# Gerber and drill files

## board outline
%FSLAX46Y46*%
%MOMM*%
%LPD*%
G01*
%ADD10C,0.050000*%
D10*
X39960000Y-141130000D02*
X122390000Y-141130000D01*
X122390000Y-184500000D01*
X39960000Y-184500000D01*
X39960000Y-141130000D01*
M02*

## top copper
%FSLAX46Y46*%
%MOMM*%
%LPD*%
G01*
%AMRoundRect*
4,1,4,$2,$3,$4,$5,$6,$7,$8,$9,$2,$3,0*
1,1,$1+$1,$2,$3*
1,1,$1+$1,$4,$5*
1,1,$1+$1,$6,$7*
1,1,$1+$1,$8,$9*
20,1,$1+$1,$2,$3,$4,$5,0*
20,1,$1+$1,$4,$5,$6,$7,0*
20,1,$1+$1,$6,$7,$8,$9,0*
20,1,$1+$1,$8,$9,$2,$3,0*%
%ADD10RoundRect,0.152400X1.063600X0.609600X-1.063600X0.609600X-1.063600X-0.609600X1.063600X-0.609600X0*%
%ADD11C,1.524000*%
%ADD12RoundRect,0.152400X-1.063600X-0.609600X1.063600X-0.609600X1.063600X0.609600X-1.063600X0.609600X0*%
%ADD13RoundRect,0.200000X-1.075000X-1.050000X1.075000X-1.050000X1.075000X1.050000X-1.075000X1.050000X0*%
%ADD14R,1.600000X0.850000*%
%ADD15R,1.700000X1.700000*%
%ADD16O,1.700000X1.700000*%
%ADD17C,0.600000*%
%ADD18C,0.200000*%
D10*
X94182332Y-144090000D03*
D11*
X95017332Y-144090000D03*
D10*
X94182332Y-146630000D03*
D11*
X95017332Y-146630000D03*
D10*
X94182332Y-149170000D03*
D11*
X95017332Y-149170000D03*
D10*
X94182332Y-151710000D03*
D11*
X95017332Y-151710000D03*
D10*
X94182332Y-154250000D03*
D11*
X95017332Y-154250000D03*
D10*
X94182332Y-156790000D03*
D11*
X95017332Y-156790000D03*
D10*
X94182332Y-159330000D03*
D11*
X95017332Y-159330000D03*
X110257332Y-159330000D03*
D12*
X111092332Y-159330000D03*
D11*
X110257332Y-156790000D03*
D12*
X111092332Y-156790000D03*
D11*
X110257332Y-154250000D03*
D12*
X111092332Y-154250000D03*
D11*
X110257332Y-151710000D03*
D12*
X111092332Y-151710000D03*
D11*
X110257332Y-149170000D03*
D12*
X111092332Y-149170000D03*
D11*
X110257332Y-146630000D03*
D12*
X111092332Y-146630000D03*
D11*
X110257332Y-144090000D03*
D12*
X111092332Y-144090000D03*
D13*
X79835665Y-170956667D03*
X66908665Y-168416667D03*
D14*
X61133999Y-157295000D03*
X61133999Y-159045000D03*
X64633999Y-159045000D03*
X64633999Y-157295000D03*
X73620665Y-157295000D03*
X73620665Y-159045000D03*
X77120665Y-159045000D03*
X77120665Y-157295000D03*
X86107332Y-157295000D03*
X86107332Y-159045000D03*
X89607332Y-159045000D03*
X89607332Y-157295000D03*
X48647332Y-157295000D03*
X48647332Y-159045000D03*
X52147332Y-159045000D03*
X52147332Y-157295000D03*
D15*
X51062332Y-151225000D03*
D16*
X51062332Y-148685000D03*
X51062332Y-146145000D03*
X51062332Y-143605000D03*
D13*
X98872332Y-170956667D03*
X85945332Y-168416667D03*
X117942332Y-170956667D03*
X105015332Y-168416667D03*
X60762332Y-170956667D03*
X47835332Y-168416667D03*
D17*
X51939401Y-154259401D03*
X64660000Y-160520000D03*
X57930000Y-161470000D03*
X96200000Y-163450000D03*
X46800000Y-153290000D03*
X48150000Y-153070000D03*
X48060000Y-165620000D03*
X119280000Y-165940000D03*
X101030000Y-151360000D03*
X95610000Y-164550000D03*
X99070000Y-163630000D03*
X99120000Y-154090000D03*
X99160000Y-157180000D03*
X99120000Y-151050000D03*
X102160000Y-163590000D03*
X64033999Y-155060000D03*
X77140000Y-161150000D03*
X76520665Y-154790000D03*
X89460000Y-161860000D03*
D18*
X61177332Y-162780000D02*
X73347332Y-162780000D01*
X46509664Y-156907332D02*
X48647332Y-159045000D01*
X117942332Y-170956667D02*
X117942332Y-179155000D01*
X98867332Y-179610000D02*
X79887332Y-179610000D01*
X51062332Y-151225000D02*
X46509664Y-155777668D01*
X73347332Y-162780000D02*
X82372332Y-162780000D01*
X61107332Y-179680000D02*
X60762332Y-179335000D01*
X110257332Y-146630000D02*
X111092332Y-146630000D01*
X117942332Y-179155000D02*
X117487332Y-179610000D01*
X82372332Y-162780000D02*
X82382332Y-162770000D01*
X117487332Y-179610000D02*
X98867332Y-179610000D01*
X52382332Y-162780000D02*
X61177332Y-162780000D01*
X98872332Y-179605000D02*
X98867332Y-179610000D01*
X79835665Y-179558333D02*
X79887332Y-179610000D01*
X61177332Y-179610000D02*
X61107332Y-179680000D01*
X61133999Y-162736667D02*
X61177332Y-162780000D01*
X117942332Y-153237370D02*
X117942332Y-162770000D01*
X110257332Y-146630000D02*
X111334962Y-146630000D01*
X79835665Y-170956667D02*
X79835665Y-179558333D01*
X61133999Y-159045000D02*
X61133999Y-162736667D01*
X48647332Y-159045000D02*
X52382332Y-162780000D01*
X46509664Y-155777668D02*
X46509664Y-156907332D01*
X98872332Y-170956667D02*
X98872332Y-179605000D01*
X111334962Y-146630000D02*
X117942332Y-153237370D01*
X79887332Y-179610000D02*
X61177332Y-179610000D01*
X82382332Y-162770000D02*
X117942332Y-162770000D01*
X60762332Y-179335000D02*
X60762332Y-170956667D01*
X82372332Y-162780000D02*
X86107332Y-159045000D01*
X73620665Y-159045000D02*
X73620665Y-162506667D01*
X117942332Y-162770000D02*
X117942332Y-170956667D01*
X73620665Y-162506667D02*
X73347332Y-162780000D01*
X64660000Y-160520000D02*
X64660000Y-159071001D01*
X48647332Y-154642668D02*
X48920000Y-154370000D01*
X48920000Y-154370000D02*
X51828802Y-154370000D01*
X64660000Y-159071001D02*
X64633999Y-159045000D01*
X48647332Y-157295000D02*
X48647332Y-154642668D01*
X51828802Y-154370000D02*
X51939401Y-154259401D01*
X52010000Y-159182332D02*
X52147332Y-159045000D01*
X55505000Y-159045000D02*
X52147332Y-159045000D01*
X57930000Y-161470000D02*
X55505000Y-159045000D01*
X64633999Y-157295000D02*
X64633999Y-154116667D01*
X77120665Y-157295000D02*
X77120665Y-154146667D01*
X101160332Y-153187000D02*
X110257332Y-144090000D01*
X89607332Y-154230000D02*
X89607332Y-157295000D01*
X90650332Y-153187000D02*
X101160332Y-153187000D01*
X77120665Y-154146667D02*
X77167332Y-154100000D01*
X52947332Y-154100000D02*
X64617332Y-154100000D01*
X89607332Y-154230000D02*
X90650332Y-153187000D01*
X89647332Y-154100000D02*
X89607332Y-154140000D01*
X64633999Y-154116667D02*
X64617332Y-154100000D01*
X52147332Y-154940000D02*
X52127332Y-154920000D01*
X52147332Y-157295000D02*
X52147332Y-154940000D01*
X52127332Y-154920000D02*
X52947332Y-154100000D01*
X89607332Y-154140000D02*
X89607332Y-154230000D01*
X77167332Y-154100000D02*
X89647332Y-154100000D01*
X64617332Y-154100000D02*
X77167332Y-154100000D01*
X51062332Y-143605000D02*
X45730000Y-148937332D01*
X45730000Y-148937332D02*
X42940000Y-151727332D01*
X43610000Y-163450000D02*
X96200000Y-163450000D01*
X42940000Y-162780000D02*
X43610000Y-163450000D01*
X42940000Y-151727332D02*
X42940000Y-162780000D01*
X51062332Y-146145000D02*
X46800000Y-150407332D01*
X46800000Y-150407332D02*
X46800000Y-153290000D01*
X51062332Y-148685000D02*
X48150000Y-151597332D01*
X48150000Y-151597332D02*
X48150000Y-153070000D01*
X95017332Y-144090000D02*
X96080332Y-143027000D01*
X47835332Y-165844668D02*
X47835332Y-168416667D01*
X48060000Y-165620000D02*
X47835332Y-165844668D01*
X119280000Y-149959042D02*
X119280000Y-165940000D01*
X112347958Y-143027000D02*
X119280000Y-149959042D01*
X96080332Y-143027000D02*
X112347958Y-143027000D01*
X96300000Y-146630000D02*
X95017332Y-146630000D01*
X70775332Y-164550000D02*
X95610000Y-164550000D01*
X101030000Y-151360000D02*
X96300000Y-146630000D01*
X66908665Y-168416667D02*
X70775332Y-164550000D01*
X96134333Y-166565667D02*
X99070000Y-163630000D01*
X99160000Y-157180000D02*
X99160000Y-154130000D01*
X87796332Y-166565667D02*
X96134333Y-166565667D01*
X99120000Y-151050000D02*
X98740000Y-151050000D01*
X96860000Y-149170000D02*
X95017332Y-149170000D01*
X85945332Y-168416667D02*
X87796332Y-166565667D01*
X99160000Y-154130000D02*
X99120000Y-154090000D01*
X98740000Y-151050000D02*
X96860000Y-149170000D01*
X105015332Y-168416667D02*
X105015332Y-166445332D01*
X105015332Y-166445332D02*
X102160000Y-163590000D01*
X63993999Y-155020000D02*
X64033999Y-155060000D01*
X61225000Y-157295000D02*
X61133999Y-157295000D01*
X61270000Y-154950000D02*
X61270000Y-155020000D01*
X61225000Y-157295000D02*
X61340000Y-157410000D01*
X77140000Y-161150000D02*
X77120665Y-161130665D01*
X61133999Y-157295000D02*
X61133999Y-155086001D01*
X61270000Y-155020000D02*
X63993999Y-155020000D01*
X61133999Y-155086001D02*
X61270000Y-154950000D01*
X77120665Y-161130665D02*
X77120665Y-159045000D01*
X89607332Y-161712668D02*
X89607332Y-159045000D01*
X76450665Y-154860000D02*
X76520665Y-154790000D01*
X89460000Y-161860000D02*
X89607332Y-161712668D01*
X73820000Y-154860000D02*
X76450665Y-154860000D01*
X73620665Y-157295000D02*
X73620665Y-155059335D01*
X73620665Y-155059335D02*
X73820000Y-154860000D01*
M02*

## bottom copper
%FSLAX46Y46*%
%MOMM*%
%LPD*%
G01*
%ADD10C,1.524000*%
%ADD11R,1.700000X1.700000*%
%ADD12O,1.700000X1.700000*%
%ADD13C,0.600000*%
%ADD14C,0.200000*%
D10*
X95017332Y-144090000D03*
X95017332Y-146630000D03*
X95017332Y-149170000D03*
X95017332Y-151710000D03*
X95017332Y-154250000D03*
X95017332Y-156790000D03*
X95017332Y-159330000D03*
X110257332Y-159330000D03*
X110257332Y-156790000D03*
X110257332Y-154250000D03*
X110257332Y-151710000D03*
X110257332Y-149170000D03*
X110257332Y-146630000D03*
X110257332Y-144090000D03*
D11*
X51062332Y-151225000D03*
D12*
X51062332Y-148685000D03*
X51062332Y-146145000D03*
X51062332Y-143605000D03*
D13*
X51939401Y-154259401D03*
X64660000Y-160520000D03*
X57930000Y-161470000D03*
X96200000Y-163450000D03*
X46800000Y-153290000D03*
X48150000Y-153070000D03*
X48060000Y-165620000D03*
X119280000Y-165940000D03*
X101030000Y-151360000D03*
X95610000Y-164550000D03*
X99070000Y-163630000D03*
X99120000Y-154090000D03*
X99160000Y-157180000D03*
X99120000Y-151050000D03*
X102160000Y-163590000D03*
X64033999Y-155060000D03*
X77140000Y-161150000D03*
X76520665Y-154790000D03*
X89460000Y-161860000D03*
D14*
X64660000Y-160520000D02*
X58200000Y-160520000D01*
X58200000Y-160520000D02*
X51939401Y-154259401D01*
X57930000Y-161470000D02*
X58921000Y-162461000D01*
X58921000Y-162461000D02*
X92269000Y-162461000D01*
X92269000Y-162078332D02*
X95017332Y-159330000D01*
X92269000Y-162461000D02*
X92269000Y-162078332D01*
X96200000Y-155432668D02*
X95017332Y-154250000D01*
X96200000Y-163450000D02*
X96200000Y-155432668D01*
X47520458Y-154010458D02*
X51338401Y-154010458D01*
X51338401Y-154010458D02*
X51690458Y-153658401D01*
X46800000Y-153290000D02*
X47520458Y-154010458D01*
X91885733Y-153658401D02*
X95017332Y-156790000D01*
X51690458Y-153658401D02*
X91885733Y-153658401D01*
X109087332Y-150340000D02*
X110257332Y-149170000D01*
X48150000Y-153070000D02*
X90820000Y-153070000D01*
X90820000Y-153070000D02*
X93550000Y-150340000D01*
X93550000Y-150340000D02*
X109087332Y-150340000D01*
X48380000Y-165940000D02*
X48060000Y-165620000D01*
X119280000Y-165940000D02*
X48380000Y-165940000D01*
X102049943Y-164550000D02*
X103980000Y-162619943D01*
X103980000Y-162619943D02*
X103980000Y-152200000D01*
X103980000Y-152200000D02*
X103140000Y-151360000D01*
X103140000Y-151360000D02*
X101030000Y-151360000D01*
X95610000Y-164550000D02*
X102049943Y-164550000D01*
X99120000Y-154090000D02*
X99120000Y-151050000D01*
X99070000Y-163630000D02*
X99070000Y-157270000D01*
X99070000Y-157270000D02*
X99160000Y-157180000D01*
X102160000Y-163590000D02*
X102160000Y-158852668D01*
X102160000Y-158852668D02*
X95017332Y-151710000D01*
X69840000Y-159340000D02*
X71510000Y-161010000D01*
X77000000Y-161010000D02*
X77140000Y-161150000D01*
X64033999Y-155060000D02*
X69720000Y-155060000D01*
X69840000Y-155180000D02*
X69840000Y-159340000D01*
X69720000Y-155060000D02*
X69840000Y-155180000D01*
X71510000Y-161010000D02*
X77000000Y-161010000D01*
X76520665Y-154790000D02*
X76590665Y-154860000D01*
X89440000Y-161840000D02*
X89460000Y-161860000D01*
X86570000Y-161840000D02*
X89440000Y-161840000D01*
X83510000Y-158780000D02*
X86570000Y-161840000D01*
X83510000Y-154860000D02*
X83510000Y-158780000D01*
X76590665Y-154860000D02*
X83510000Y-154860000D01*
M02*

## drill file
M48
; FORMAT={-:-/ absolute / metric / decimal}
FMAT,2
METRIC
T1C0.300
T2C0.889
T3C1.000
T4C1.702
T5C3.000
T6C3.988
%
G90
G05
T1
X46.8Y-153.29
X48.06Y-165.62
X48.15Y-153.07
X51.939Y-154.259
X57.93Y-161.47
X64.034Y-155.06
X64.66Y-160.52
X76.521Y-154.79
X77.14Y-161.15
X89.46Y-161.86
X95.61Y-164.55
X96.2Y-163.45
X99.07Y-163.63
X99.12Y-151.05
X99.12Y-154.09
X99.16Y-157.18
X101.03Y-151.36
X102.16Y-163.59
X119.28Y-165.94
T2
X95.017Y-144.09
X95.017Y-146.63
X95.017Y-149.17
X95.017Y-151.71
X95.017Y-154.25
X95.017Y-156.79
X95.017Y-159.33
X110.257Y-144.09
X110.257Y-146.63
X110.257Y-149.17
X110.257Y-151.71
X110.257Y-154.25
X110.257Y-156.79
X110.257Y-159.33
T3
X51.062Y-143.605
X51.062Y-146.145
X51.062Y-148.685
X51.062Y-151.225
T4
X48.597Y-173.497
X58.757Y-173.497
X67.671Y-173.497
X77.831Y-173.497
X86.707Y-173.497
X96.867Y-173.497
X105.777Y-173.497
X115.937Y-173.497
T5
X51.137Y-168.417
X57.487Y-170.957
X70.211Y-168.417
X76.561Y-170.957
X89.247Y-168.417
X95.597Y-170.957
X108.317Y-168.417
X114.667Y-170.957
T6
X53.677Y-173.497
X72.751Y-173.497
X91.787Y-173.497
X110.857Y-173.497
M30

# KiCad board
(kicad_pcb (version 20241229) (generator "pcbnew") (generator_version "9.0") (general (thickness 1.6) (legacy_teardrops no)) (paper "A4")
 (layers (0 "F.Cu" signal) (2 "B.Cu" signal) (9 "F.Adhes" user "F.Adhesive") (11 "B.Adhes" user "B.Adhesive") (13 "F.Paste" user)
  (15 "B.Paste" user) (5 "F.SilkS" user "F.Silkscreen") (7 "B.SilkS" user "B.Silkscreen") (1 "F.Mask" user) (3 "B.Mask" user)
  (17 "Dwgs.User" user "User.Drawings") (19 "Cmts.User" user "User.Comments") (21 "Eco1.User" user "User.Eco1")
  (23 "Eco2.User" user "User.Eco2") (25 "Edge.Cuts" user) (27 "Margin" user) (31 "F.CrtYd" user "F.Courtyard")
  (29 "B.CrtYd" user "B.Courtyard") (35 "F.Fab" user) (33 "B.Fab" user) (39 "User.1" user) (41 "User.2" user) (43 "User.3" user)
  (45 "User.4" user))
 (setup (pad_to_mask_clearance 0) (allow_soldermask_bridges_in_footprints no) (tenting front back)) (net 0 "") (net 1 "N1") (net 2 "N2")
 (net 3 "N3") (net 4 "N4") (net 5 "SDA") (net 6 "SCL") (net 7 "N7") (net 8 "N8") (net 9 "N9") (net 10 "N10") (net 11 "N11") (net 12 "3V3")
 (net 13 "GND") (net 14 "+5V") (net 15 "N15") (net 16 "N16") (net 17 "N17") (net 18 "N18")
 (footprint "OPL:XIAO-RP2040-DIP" (layer "F.Cu") (at 102.637332 151.71)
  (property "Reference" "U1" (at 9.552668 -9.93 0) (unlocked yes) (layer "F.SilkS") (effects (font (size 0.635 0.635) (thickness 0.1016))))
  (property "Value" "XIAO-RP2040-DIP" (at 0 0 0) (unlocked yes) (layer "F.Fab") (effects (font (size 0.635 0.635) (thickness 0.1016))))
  (pad "1" smd roundrect (at -8.455 -7.62 180) (size 2.432 1.524) (layers "F.Cu" "F.Mask") (roundrect_rratio 0.1) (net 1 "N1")
   (thermal_bridge_angle 45))
  (pad "1" thru_hole circle (at -7.62 -7.62 180) (size 1.524 1.524) (drill 0.889) (layers "*.Cu" "*.Mask") (remove_unused_layers no)
   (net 1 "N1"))
  (pad "2" smd roundrect (at -8.455 -5.08 180) (size 2.432 1.524) (layers "F.Cu" "F.Mask") (roundrect_rratio 0.1) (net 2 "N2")
   (thermal_bridge_angle 45))
  (pad "2" thru_hole circle (at -7.62 -5.08 180) (size 1.524 1.524) (drill 0.889) (layers "*.Cu" "*.Mask") (remove_unused_layers no)
   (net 2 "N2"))
  (pad "3" smd roundrect (at -8.455 -2.54 180) (size 2.432 1.524) (layers "F.Cu" "F.Mask") (roundrect_rratio 0.1) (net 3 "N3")
   (thermal_bridge_angle 45))
  (pad "3" thru_hole circle (at -7.62 -2.54 180) (size 1.524 1.524) (drill 0.889) (layers "*.Cu" "*.Mask") (remove_unused_layers no)
   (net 3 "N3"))
  (pad "4" smd roundrect (at -8.455 0 180) (size 2.432 1.524) (layers "F.Cu" "F.Mask") (roundrect_rratio 0.1) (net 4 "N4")
   (thermal_bridge_angle 45))
  (pad "4" thru_hole circle (at -7.62 0 180) (size 1.524 1.524) (drill 0.889) (layers "*.Cu" "*.Mask") (remove_unused_layers no)
   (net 4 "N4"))
  (pad "5" smd roundrect (at -8.455 2.54 180) (size 2.432 1.524) (layers "F.Cu" "F.Mask") (roundrect_rratio 0.1) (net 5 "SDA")
   (thermal_bridge_angle 45))
  (pad "5" thru_hole circle (at -7.62 2.54 180) (size 1.524 1.524) (drill 0.889) (layers "*.Cu" "*.Mask") (remove_unused_layers no)
   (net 5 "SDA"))
  (pad "6" smd roundrect (at -8.455 5.08 180) (size 2.432 1.524) (layers "F.Cu" "F.Mask") (roundrect_rratio 0.1) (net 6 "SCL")
   (thermal_bridge_angle 45))
  (pad "6" thru_hole circle (at -7.62 5.08 180) (size 1.524 1.524) (drill 0.889) (layers "*.Cu" "*.Mask") (remove_unused_layers no)
   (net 6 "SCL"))
  (pad "7" smd roundrect (at -8.455 7.62 180) (size 2.432 1.524) (layers "F.Cu" "F.Mask") (roundrect_rratio 0.1) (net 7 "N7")
   (thermal_bridge_angle 45))
  (pad "7" thru_hole circle (at -7.62 7.62 180) (size 1.524 1.524) (drill 0.889) (layers "*.Cu" "*.Mask") (remove_unused_layers no)
   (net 7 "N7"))
  (pad "8" thru_hole circle (at 7.62 7.62) (size 1.524 1.524) (drill 0.889) (layers "*.Cu" "*.Mask") (remove_unused_layers no) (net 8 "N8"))
  (pad "8" smd roundrect (at 8.455 7.62) (size 2.432 1.524) (layers "F.Cu" "F.Mask") (roundrect_rratio 0.1) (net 8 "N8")
   (thermal_bridge_angle 45))
  (pad "9" thru_hole circle (at 7.62 5.08) (size 1.524 1.524) (drill 0.889) (layers "*.Cu" "*.Mask") (remove_unused_layers no) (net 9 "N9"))
  (pad "9" smd roundrect (at 8.455 5.08) (size 2.432 1.524) (layers "F.Cu" "F.Mask") (roundrect_rratio 0.1) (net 9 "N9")
   (thermal_bridge_angle 45))
  (pad "10" thru_hole circle (at 7.62 2.54) (size 1.524 1.524) (drill 0.889) (layers "*.Cu" "*.Mask") (remove_unused_layers no)
   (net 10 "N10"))
  (pad "10" smd roundrect (at 8.455 2.54) (size 2.432 1.524) (layers "F.Cu" "F.Mask") (roundrect_rratio 0.1) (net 10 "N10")
   (thermal_bridge_angle 45))
  (pad "11" thru_hole circle (at 7.62 0) (size 1.524 1.524) (drill 0.889) (layers "*.Cu" "*.Mask") (remove_unused_layers no) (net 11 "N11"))
  (pad "11" smd roundrect (at 8.455 0) (size 2.432 1.524) (layers "F.Cu" "F.Mask") (roundrect_rratio 0.1) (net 11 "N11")
   (thermal_bridge_angle 45))
  (pad "12" thru_hole circle (at 7.62 -2.54) (size 1.524 1.524) (drill 0.889) (layers "*.Cu" "*.Mask") (remove_unused_layers no)
   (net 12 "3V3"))
  (pad "12" smd roundrect (at 8.455 -2.54) (size 2.432 1.524) (layers "F.Cu" "F.Mask") (roundrect_rratio 0.1) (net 12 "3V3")
   (thermal_bridge_angle 45))
  (pad "13" thru_hole circle (at 7.62 -5.08) (size 1.524 1.524) (drill 0.889) (layers "*.Cu" "*.Mask") (remove_unused_layers no)
   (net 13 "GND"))
  (pad "13" smd roundrect (at 8.455 -5.08) (size 2.432 1.524) (layers "F.Cu" "F.Mask") (roundrect_rratio 0.1) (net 13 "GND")
   (thermal_bridge_angle 45))
  (pad "14" thru_hole circle (at 7.62 -7.62) (size 1.524 1.524) (drill 0.889) (layers "*.Cu" "*.Mask") (remove_unused_layers no)
   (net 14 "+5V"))
  (pad "14" smd roundrect (at 8.455 -7.62) (size 2.432 1.524) (layers "F.Cu" "F.Mask") (roundrect_rratio 0.1) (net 14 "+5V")
   (thermal_bridge_angle 45)))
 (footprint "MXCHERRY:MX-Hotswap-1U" (layer "F.Cu") (at 72.750665 173.496667)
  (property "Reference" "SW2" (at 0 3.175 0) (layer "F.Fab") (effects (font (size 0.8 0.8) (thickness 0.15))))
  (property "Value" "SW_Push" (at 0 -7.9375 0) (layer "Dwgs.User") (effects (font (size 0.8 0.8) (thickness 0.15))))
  (pad "" np_thru_hole circle (at -5.08 0 311.901) (size 1.7018 1.7018) (drill 1.7018) (layers "*.Cu" "*.Mask"))
  (pad "" np_thru_hole circle (at -2.54 -5.08) (size 3 3) (drill 3) (layers "*.Cu" "*.Mask"))
  (pad "" np_thru_hole circle (at 0 0) (size 3.9878 3.9878) (drill 3.9878) (layers "*.Cu" "*.Mask"))
  (pad "" np_thru_hole circle (at 3.81 -2.54) (size 3 3) (drill 3) (layers "*.Cu" "*.Mask"))
  (pad "" np_thru_hole circle (at 5.08 0 311.901) (size 1.7018 1.7018) (drill 1.7018) (layers "*.Cu" "*.Mask"))
  (pad "1" smd roundrect (at 7.085 -2.54) (size 2.55 2.5) (layers "F.Cu" "F.Mask" "F.Paste") (roundrect_rratio 0.08) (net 13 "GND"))
  (pad "2" smd roundrect (at -5.842 -5.08) (size 2.55 2.5) (layers "F.Cu" "F.Mask" "F.Paste") (roundrect_rratio 0.08) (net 2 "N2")))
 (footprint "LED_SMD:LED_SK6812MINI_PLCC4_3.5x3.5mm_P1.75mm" (layer "F.Cu") (at 62.883999 158.17)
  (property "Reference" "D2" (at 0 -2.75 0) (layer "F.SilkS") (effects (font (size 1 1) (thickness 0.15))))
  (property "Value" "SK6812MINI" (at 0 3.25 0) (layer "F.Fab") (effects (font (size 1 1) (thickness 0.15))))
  (pad "1" smd rect (at -1.75 -0.875) (size 1.6 0.85) (layers "F.Cu" "F.Mask" "F.Paste") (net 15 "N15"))
  (pad "2" smd rect (at -1.75 0.875) (size 1.6 0.85) (layers "F.Cu" "F.Mask" "F.Paste") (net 13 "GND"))
  (pad "3" smd rect (at 1.75 0.875) (size 1.6 0.85) (layers "F.Cu" "F.Mask" "F.Paste") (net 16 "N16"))
  (pad "4" smd rect (at 1.75 -0.875) (size 1.6 0.85) (layers "F.Cu" "F.Mask" "F.Paste") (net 14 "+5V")))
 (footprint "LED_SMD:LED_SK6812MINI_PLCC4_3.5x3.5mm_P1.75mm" (layer "F.Cu") (at 75.370665 158.17)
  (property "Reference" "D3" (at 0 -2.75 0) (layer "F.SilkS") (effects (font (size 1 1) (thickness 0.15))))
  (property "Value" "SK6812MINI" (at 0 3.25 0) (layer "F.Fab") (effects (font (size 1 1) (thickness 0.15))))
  (pad "1" smd rect (at -1.75 -0.875) (size 1.6 0.85) (layers "F.Cu" "F.Mask" "F.Paste") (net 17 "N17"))
  (pad "2" smd rect (at -1.75 0.875) (size 1.6 0.85) (layers "F.Cu" "F.Mask" "F.Paste") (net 13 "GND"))
  (pad "3" smd rect (at 1.75 0.875) (size 1.6 0.85) (layers "F.Cu" "F.Mask" "F.Paste") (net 15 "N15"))
  (pad "4" smd rect (at 1.75 -0.875) (size 1.6 0.85) (layers "F.Cu" "F.Mask" "F.Paste") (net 14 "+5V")))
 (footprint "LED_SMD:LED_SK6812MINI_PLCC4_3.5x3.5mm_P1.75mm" (layer "F.Cu") (at 87.857332 158.17)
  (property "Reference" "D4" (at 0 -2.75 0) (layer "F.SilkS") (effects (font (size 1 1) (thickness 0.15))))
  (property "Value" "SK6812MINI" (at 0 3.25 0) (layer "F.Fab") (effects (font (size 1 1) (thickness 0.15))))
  (pad "1" smd rect (at -1.75 -0.875) (size 1.6 0.85) (layers "F.Cu" "F.Mask" "F.Paste") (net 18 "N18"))
  (pad "2" smd rect (at -1.75 0.875) (size 1.6 0.85) (layers "F.Cu" "F.Mask" "F.Paste") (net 13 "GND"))
  (pad "3" smd rect (at 1.75 0.875) (size 1.6 0.85) (layers "F.Cu" "F.Mask" "F.Paste") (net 17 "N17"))
  (pad "4" smd rect (at 1.75 -0.875) (size 1.6 0.85) (layers "F.Cu" "F.Mask" "F.Paste") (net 14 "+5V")))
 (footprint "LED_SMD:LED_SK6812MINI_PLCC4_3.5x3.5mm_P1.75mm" (layer "F.Cu") (at 50.397332 158.17)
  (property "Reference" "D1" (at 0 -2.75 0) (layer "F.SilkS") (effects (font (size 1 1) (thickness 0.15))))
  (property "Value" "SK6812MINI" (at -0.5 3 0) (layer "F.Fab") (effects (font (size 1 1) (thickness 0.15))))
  (pad "1" smd rect (at -1.75 -0.875) (size 1.6 0.85) (layers "F.Cu" "F.Mask" "F.Paste") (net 16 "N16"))
  (pad "2" smd rect (at -1.75 0.875) (size 1.6 0.85) (layers "F.Cu" "F.Mask" "F.Paste") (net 13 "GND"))
  (pad "3" smd rect (at 1.75 0.875) (size 1.6 0.85) (layers "F.Cu" "F.Mask" "F.Paste") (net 7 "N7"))
  (pad "4" smd rect (at 1.75 -0.875) (size 1.6 0.85) (layers "F.Cu" "F.Mask" "F.Paste") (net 14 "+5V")))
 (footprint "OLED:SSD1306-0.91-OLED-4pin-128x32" (layer "F.Cu") (at 87.562332 153.415 180)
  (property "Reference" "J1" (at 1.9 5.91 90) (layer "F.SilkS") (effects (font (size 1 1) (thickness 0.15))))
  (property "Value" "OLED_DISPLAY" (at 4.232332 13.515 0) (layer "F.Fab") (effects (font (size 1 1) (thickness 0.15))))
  (pad "1" thru_hole rect (at 36.5 2.19 180) (size 1.7 1.7) (drill 1) (layers "*.Cu" "*.Mask") (remove_unused_layers no) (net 13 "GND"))
  (pad "2" thru_hole oval (at 36.5 4.73 180) (size 1.7 1.7) (drill 1) (layers "*.Cu" "*.Mask") (remove_unused_layers no) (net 12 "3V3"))
  (pad "3" thru_hole oval (at 36.5 7.27 180) (size 1.7 1.7) (drill 1) (layers "*.Cu" "*.Mask") (remove_unused_layers no) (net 6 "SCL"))
  (pad "4" thru_hole oval (at 36.5 9.81 180) (size 1.7 1.7) (drill 1) (layers "*.Cu" "*.Mask") (remove_unused_layers no) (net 5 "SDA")))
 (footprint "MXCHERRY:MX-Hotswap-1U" (layer "F.Cu") (at 91.787332 173.496667)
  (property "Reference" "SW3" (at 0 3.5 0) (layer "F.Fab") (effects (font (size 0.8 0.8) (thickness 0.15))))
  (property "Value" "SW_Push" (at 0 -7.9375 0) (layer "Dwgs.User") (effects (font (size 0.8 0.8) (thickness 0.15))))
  (pad "" np_thru_hole circle (at -5.08 0 311.901) (size 1.7018 1.7018) (drill 1.7018) (layers "*.Cu" "*.Mask"))
  (pad "" np_thru_hole circle (at -2.54 -5.08) (size 3 3) (drill 3) (layers "*.Cu" "*.Mask"))
  (pad "" np_thru_hole circle (at 0 0) (size 3.9878 3.9878) (drill 3.9878) (layers "*.Cu" "*.Mask"))
  (pad "" np_thru_hole circle (at 3.81 -2.54) (size 3 3) (drill 3) (layers "*.Cu" "*.Mask"))
  (pad "" np_thru_hole circle (at 5.08 0 311.901) (size 1.7018 1.7018) (drill 1.7018) (layers "*.Cu" "*.Mask"))
  (pad "1" smd roundrect (at 7.085 -2.54) (size 2.55 2.5) (layers "F.Cu" "F.Mask" "F.Paste") (roundrect_rratio 0.08) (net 13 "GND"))
  (pad "2" smd roundrect (at -5.842 -5.08) (size 2.55 2.5) (layers "F.Cu" "F.Mask" "F.Paste") (roundrect_rratio 0.08) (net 3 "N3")))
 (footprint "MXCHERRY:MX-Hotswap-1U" (layer "F.Cu") (at 110.857332 173.496667)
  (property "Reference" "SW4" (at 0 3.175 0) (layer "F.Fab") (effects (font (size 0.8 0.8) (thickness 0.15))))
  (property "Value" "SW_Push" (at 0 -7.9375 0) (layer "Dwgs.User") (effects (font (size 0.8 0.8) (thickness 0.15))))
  (pad "" np_thru_hole circle (at -5.08 0 311.901) (size 1.7018 1.7018) (drill 1.7018) (layers "*.Cu" "*.Mask"))
  (pad "" np_thru_hole circle (at -2.54 -5.08) (size 3 3) (drill 3) (layers "*.Cu" "*.Mask"))
  (pad "" np_thru_hole circle (at 0 0) (size 3.9878 3.9878) (drill 3.9878) (layers "*.Cu" "*.Mask"))
  (pad "" np_thru_hole circle (at 3.81 -2.54) (size 3 3) (drill 3) (layers "*.Cu" "*.Mask"))
  (pad "" np_thru_hole circle (at 5.08 0 311.901) (size 1.7018 1.7018) (drill 1.7018) (layers "*.Cu" "*.Mask"))
  (pad "1" smd roundrect (at 7.085 -2.54) (size 2.55 2.5) (layers "F.Cu" "F.Mask" "F.Paste") (roundrect_rratio 0.08) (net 13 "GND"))
  (pad "2" smd roundrect (at -5.842 -5.08) (size 2.55 2.5) (layers "F.Cu" "F.Mask" "F.Paste") (roundrect_rratio 0.08) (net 4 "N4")))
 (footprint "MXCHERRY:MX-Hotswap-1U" (layer "F.Cu") (at 53.677332 173.496667)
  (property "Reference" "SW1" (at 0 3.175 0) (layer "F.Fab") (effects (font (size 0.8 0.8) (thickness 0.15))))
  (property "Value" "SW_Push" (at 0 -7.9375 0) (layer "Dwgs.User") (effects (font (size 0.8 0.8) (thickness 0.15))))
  (pad "" np_thru_hole circle (at -5.08 0 311.901) (size 1.7018 1.7018) (drill 1.7018) (layers "*.Cu" "*.Mask"))
  (pad "" np_thru_hole circle (at -2.54 -5.08) (size 3 3) (drill 3) (layers "*.Cu" "*.Mask"))
  (pad "" np_thru_hole circle (at 0 0) (size 3.9878 3.9878) (drill 3.9878) (layers "*.Cu" "*.Mask"))
  (pad "" np_thru_hole circle (at 3.81 -2.54) (size 3 3) (drill 3) (layers "*.Cu" "*.Mask"))
  (pad "" np_thru_hole circle (at 5.08 0 311.901) (size 1.7018 1.7018) (drill 1.7018) (layers "*.Cu" "*.Mask"))
  (pad "1" smd roundrect (at 7.085 -2.54) (size 2.55 2.5) (layers "F.Cu" "F.Mask" "F.Paste") (roundrect_rratio 0.08) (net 13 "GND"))
  (pad "2" smd roundrect (at -5.842 -5.08) (size 2.55 2.5) (layers "F.Cu" "F.Mask" "F.Paste") (roundrect_rratio 0.08) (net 1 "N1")))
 (gr_rect (start 39.96 141.13) (end 122.39 184.5) (stroke (width 0.05) (type default)) (fill no) (layer "Edge.Cuts"))
 (segment (start 61.177332 162.78) (end 73.347332 162.78) (width 0.2) (layer "F.Cu") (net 13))
 (segment (start 46.509664 156.907332) (end 48.647332 159.045) (width 0.2) (layer "F.Cu") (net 13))
 (segment (start 117.942332 170.956667) (end 117.942332 179.155) (width 0.2) (layer "F.Cu") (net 13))
 (segment (start 98.867332 179.61) (end 79.887332 179.61) (width 0.2) (layer "F.Cu") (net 13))
 (segment (start 51.062332 151.225) (end 46.509664 155.777668) (width 0.2) (layer "F.Cu") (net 13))
 (segment (start 73.347332 162.78) (end 82.372332 162.78) (width 0.2) (layer "F.Cu") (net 13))
 (segment (start 61.107332 179.68) (end 60.762332 179.335) (width 0.2) (layer "F.Cu") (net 13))
 (segment (start 110.257332 146.63) (end 111.092332 146.63) (width 0.2) (layer "F.Cu") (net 13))
 (segment (start 117.942332 179.155) (end 117.487332 179.61) (width 0.2) (layer "F.Cu") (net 13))
 (segment (start 82.372332 162.78) (end 82.382332 162.77) (width 0.2) (layer "F.Cu") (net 13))
 (segment (start 117.487332 179.61) (end 98.867332 179.61) (width 0.2) (layer "F.Cu") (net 13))
 (segment (start 52.382332 162.78) (end 61.177332 162.78) (width 0.2) (layer "F.Cu") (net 13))
 (segment (start 98.872332 179.605) (end 98.867332 179.61) (width 0.2) (layer "F.Cu") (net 13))
 (segment (start 79.835665 179.558333) (end 79.887332 179.61) (width 0.2) (layer "F.Cu") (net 13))
 (segment (start 61.177332 179.61) (end 61.107332 179.68) (width 0.2) (layer "F.Cu") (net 13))
 (segment (start 61.133999 162.736667) (end 61.177332 162.78) (width 0.2) (layer "F.Cu") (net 13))
 (segment (start 117.942332 153.23737) (end 117.942332 162.77) (width 0.2) (layer "F.Cu") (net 13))
 (segment (start 110.257332 146.63) (end 111.334962 146.63) (width 0.2) (layer "F.Cu") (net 13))
 (segment (start 79.835665 170.956667) (end 79.835665 179.558333) (width 0.2) (layer "F.Cu") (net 13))
 (segment (start 61.133999 159.045) (end 61.133999 162.736667) (width 0.2) (layer "F.Cu") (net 13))
 (segment (start 48.647332 159.045) (end 52.382332 162.78) (width 0.2) (layer "F.Cu") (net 13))
 (segment (start 46.509664 155.777668) (end 46.509664 156.907332) (width 0.2) (layer "F.Cu") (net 13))
 (segment (start 98.872332 170.956667) (end 98.872332 179.605) (width 0.2) (layer "F.Cu") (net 13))
 (segment (start 111.334962 146.63) (end 117.942332 153.23737) (width 0.2) (layer "F.Cu") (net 13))
 (segment (start 79.887332 179.61) (end 61.177332 179.61) (width 0.2) (layer "F.Cu") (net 13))
 (segment (start 82.382332 162.77) (end 117.942332 162.77) (width 0.2) (layer "F.Cu") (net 13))
 (segment (start 60.762332 179.335) (end 60.762332 170.956667) (width 0.2) (layer "F.Cu") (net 13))
 (segment (start 82.372332 162.78) (end 86.107332 159.045) (width 0.2) (layer "F.Cu") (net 13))
 (segment (start 73.620665 159.045) (end 73.620665 162.506667) (width 0.2) (layer "F.Cu") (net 13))
 (segment (start 117.942332 162.77) (end 117.942332 170.956667) (width 0.2) (layer "F.Cu") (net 13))
 (segment (start 73.620665 162.506667) (end 73.347332 162.78) (width 0.2) (layer "F.Cu") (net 13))
 (segment (start 64.66 160.52) (end 64.66 159.071001) (width 0.2) (layer "F.Cu") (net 16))
 (segment (start 48.647332 154.642668) (end 48.92 154.37) (width 0.2) (layer "F.Cu") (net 16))
 (segment (start 48.92 154.37) (end 51.828802 154.37) (width 0.2) (layer "F.Cu") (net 16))
 (segment (start 64.66 159.071001) (end 64.633999 159.045) (width 0.2) (layer "F.Cu") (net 16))
 (segment (start 48.647332 157.295) (end 48.647332 154.642668) (width 0.2) (layer "F.Cu") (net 16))
 (segment (start 51.828802 154.37) (end 51.939401 154.259401) (width 0.2) (layer "F.Cu") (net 16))
 (via (at 51.939401 154.259401) (size 0.6) (drill 0.3) (layers "F.Cu" "B.Cu") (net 16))
 (via (at 64.66 160.52) (size 0.6) (drill 0.3) (layers "F.Cu" "B.Cu") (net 16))
 (segment (start 64.66 160.52) (end 58.2 160.52) (width 0.2) (layer "B.Cu") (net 16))
 (segment (start 58.2 160.52) (end 51.939401 154.259401) (width 0.2) (layer "B.Cu") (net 16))
 (segment (start 52.01 159.182332) (end 52.147332 159.045) (width 0.2) (layer "F.Cu") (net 7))
 (segment (start 55.505 159.045) (end 52.147332 159.045) (width 0.2) (layer "F.Cu") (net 7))
 (segment (start 57.93 161.47) (end 55.505 159.045) (width 0.2) (layer "F.Cu") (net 7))
 (via (at 57.93 161.47) (size 0.6) (drill 0.3) (layers "F.Cu" "B.Cu") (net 7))
 (segment (start 57.93 161.47) (end 58.921 162.461) (width 0.2) (layer "B.Cu") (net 7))
 (segment (start 58.921 162.461) (end 92.269 162.461) (width 0.2) (layer "B.Cu") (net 7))
 (segment (start 92.269 162.078332) (end 95.017332 159.33) (width 0.2) (layer "B.Cu") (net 7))
 (segment (start 92.269 162.461) (end 92.269 162.078332) (width 0.2) (layer "B.Cu") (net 7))
 (segment (start 64.633999 157.295) (end 64.633999 154.116667) (width 0.2) (layer "F.Cu") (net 14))
 (segment (start 77.120665 157.295) (end 77.120665 154.146667) (width 0.2) (layer "F.Cu") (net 14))
 (segment (start 101.160332 153.187) (end 110.257332 144.09) (width 0.2) (layer "F.Cu") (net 14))
 (segment (start 89.607332 154.23) (end 89.607332 157.295) (width 0.2) (layer "F.Cu") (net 14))
 (segment (start 90.650332 153.187) (end 101.160332 153.187) (width 0.2) (layer "F.Cu") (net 14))
 (segment (start 77.120665 154.146667) (end 77.167332 154.1) (width 0.2) (layer "F.Cu") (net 14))
 (segment (start 52.947332 154.1) (end 64.617332 154.1) (width 0.2) (layer "F.Cu") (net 14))
 (segment (start 89.607332 154.23) (end 90.650332 153.187) (width 0.2) (layer "F.Cu") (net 14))
 (segment (start 89.647332 154.1) (end 89.607332 154.14) (width 0.2) (layer "F.Cu") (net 14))
 (segment (start 64.633999 154.116667) (end 64.617332 154.1) (width 0.2) (layer "F.Cu") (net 14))
 (segment (start 52.147332 154.94) (end 52.127332 154.92) (width 0.2) (layer "F.Cu") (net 14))
 (segment (start 52.147332 157.295) (end 52.147332 154.94) (width 0.2) (layer "F.Cu") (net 14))
 (segment (start 52.127332 154.92) (end 52.947332 154.1) (width 0.2) (layer "F.Cu") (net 14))
 (segment (start 89.607332 154.14) (end 89.607332 154.23) (width 0.2) (layer "F.Cu") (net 14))
 (segment (start 77.167332 154.1) (end 89.647332 154.1) (width 0.2) (layer "F.Cu") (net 14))
 (segment (start 64.617332 154.1) (end 77.167332 154.1) (width 0.2) (layer "F.Cu") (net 14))
 (segment (start 51.062332 143.605) (end 45.73 148.937332) (width 0.2) (layer "F.Cu") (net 5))
 (segment (start 45.73 148.937332) (end 42.94 151.727332) (width 0.2) (layer "F.Cu") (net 5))
 (segment (start 43.61 163.45) (end 96.2 163.45) (width 0.2) (layer "F.Cu") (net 5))
 (segment (start 42.94 162.78) (end 43.61 163.45) (width 0.2) (layer "F.Cu") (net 5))
 (segment (start 42.94 151.727332) (end 42.94 162.78) (width 0.2) (layer "F.Cu") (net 5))
 (via (at 96.2 163.45) (size 0.6) (drill 0.3) (layers "F.Cu" "B.Cu") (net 5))
 (segment (start 96.2 155.432668) (end 95.017332 154.25) (width 0.2) (layer "B.Cu") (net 5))
 (segment (start 96.2 163.45) (end 96.2 155.432668) (width 0.2) (layer "B.Cu") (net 5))
 (segment (start 51.062332 146.145) (end 46.8 150.407332) (width 0.2) (layer "F.Cu") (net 6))
 (segment (start 46.8 150.407332) (end 46.8 153.29) (width 0.2) (layer "F.Cu") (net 6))
 (via (at 46.8 153.29) (size 0.6) (drill 0.3) (layers "F.Cu" "B.Cu") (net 6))
 (segment (start 47.520458 154.010458) (end 51.338401 154.010458) (width 0.2) (layer "B.Cu") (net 6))
 (segment (start 51.338401 154.010458) (end 51.690458 153.658401) (width 0.2) (layer "B.Cu") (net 6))
 (segment (start 46.8 153.29) (end 47.520458 154.010458) (width 0.2) (layer "B.Cu") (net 6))
 (segment (start 91.885733 153.658401) (end 95.017332 156.79) (width 0.2) (layer "B.Cu") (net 6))
 (segment (start 51.690458 153.658401) (end 91.885733 153.658401) (width 0.2) (layer "B.Cu") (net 6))
 (segment (start 51.062332 148.685) (end 48.15 151.597332) (width 0.2) (layer "F.Cu") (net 12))
 (segment (start 48.15 151.597332) (end 48.15 153.07) (width 0.2) (layer "F.Cu") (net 12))
 (via (at 48.15 153.07) (size 0.6) (drill 0.3) (layers "F.Cu" "B.Cu") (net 12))
 (segment (start 109.087332 150.34) (end 110.257332 149.17) (width 0.2) (layer "B.Cu") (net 12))
 (segment (start 48.15 153.07) (end 90.82 153.07) (width 0.2) (layer "B.Cu") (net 12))
 (segment (start 90.82 153.07) (end 93.55 150.34) (width 0.2) (layer "B.Cu") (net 12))
 (segment (start 93.55 150.34) (end 109.087332 150.34) (width 0.2) (layer "B.Cu") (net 12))
 (segment (start 95.017332 144.09) (end 96.080332 143.027) (width 0.2) (layer "F.Cu") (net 1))
 (segment (start 47.835332 165.844668) (end 47.835332 168.416667) (width 0.2) (layer "F.Cu") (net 1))
 (segment (start 48.06 165.62) (end 47.835332 165.844668) (width 0.2) (layer "F.Cu") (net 1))
 (segment (start 119.28 149.959042) (end 119.28 165.94) (width 0.2) (layer "F.Cu") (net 1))
 (segment (start 112.347958 143.027) (end 119.28 149.959042) (width 0.2) (layer "F.Cu") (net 1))
 (segment (start 96.080332 143.027) (end 112.347958 143.027) (width 0.2) (layer "F.Cu") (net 1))
 (via (at 48.06 165.62) (size 0.6) (drill 0.3) (layers "F.Cu" "B.Cu") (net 1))
 (via (at 119.28 165.94) (size 0.6) (drill 0.3) (layers "F.Cu" "B.Cu") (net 1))
 (segment (start 48.38 165.94) (end 48.06 165.62) (width 0.2) (layer "B.Cu") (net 1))
 (segment (start 119.28 165.94) (end 48.38 165.94) (width 0.2) (layer "B.Cu") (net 1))
 (segment (start 96.3 146.63) (end 95.017332 146.63) (width 0.2) (layer "F.Cu") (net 2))
 (segment (start 70.775332 164.55) (end 95.61 164.55) (width 0.2) (layer "F.Cu") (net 2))
 (segment (start 101.03 151.36) (end 96.3 146.63) (width 0.2) (layer "F.Cu") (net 2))
 (segment (start 66.908665 168.416667) (end 70.775332 164.55) (width 0.2) (layer "F.Cu") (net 2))
 (via (at 101.03 151.36) (size 0.6) (drill 0.3) (layers "F.Cu" "B.Cu") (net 2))
 (via (at 95.61 164.55) (size 0.6) (drill 0.3) (layers "F.Cu" "B.Cu") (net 2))
 (segment (start 102.049943 164.55) (end 103.98 162.619943) (width 0.2) (layer "B.Cu") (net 2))
 (segment (start 103.98 162.619943) (end 103.98 152.2) (width 0.2) (layer "B.Cu") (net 2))
 (segment (start 103.98 152.2) (end 103.14 151.36) (width 0.2) (layer "B.Cu") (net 2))
 (segment (start 103.14 151.36) (end 101.03 151.36) (width 0.2) (layer "B.Cu") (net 2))
 (segment (start 95.61 164.55) (end 102.049943 164.55) (width 0.2) (layer "B.Cu") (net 2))
 (segment (start 96.134333 166.565667) (end 99.07 163.63) (width 0.2) (layer "F.Cu") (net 3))
 (segment (start 99.16 157.18) (end 99.16 154.13) (width 0.2) (layer "F.Cu") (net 3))
 (segment (start 87.796332 166.565667) (end 96.134333 166.565667) (width 0.2) (layer "F.Cu") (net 3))
 (segment (start 99.12 151.05) (end 98.74 151.05) (width 0.2) (layer "F.Cu") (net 3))
 (segment (start 96.86 149.17) (end 95.017332 149.17) (width 0.2) (layer "F.Cu") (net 3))
 (segment (start 85.945332 168.416667) (end 87.796332 166.565667) (width 0.2) (layer "F.Cu") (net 3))
 (segment (start 99.16 154.13) (end 99.12 154.09) (width 0.2) (layer "F.Cu") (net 3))
 (segment (start 98.74 151.05) (end 96.86 149.17) (width 0.2) (layer "F.Cu") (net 3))
 (via (at 99.07 163.63) (size 0.6) (drill 0.3) (layers "F.Cu" "B.Cu") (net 3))
 (via (at 99.12 154.09) (size 0.6) (drill 0.3) (layers "F.Cu" "B.Cu") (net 3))
 (via (at 99.16 157.18) (size 0.6) (drill 0.3) (layers "F.Cu" "B.Cu") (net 3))
 (via (at 99.12 151.05) (size 0.6) (drill 0.3) (layers "F.Cu" "B.Cu") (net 3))
 (segment (start 99.12 154.09) (end 99.12 151.05) (width 0.2) (layer "B.Cu") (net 3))
 (segment (start 99.07 163.63) (end 99.07 157.27) (width 0.2) (layer "B.Cu") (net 3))
 (segment (start 99.07 157.27) (end 99.16 157.18) (width 0.2) (layer "B.Cu") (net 3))
 (segment (start 105.015332 168.416667) (end 105.015332 166.445332) (width 0.2) (layer "F.Cu") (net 4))
 (segment (start 105.015332 166.445332) (end 102.16 163.59) (width 0.2) (layer "F.Cu") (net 4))
 (via (at 102.16 163.59) (size 0.6) (drill 0.3) (layers "F.Cu" "B.Cu") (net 4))
 (segment (start 102.16 163.59) (end 102.16 158.852668) (width 0.2) (layer "B.Cu") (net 4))
 (segment (start 102.16 158.852668) (end 95.017332 151.71) (width 0.2) (layer "B.Cu") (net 4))
 (segment (start 63.993999 155.02) (end 64.033999 155.06) (width 0.2) (layer "F.Cu") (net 15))
 (segment (start 61.225 157.295) (end 61.133999 157.295) (width 0.2) (layer "F.Cu") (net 15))
 (segment (start 61.27 154.95) (end 61.27 155.02) (width 0.2) (layer "F.Cu") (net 15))
 (segment (start 61.225 157.295) (end 61.34 157.41) (width 0.2) (layer "F.Cu") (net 15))
 (segment (start 77.14 161.15) (end 77.120665 161.130665) (width 0.2) (layer "F.Cu") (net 15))
 (segment (start 61.133999 157.295) (end 61.133999 155.086001) (width 0.2) (layer "F.Cu") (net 15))
 (segment (start 61.27 155.02) (end 63.993999 155.02) (width 0.2) (layer "F.Cu") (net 15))
 (segment (start 61.133999 155.086001) (end 61.27 154.95) (width 0.2) (layer "F.Cu") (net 15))
 (segment (start 77.120665 161.130665) (end 77.120665 159.045) (width 0.2) (layer "F.Cu") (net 15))
 (via (at 64.033999 155.06) (size 0.6) (drill 0.3) (layers "F.Cu" "B.Cu") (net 15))
 (via (at 77.14 161.15) (size 0.6) (drill 0.3) (layers "F.Cu" "B.Cu") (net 15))
 (segment (start 69.84 159.34) (end 71.51 161.01) (width 0.2) (layer "B.Cu") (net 15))
 (segment (start 77 161.01) (end 77.14 161.15) (width 0.2) (layer "B.Cu") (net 15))
 (segment (start 64.033999 155.06) (end 69.72 155.06) (width 0.2) (layer "B.Cu") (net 15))
 (segment (start 69.84 155.18) (end 69.84 159.34) (width 0.2) (layer "B.Cu") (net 15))
 (segment (start 69.72 155.06) (end 69.84 155.18) (width 0.2) (layer "B.Cu") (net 15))
 (segment (start 71.51 161.01) (end 77 161.01) (width 0.2) (layer "B.Cu") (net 15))
 (segment (start 89.607332 161.712668) (end 89.607332 159.045) (width 0.2) (layer "F.Cu") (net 17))
 (segment (start 76.450665 154.86) (end 76.520665 154.79) (width 0.2) (layer "F.Cu") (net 17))
 (segment (start 89.46 161.86) (end 89.607332 161.712668) (width 0.2) (layer "F.Cu") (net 17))
 (segment (start 73.82 154.86) (end 76.450665 154.86) (width 0.2) (layer "F.Cu") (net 17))
 (segment (start 73.620665 157.295) (end 73.620665 155.059335) (width 0.2) (layer "F.Cu") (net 17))
 (segment (start 73.620665 155.059335) (end 73.82 154.86) (width 0.2) (layer "F.Cu") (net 17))
 (via (at 76.520665 154.79) (size 0.6) (drill 0.3) (layers "F.Cu" "B.Cu") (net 17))
 (via (at 89.46 161.86) (size 0.6) (drill 0.3) (layers "F.Cu" "B.Cu") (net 17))
 (segment (start 76.520665 154.79) (end 76.590665 154.86) (width 0.2) (layer "B.Cu") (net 17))
 (segment (start 89.44 161.84) (end 89.46 161.86) (width 0.2) (layer "B.Cu") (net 17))
 (segment (start 86.57 161.84) (end 89.44 161.84) (width 0.2) (layer "B.Cu") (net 17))
 (segment (start 83.51 158.78) (end 86.57 161.84) (width 0.2) (layer "B.Cu") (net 17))
 (segment (start 83.51 154.86) (end 83.51 158.78) (width 0.2) (layer "B.Cu") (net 17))
 (segment (start 76.590665 154.86) (end 83.51 154.86) (width 0.2) (layer "B.Cu") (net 17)))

